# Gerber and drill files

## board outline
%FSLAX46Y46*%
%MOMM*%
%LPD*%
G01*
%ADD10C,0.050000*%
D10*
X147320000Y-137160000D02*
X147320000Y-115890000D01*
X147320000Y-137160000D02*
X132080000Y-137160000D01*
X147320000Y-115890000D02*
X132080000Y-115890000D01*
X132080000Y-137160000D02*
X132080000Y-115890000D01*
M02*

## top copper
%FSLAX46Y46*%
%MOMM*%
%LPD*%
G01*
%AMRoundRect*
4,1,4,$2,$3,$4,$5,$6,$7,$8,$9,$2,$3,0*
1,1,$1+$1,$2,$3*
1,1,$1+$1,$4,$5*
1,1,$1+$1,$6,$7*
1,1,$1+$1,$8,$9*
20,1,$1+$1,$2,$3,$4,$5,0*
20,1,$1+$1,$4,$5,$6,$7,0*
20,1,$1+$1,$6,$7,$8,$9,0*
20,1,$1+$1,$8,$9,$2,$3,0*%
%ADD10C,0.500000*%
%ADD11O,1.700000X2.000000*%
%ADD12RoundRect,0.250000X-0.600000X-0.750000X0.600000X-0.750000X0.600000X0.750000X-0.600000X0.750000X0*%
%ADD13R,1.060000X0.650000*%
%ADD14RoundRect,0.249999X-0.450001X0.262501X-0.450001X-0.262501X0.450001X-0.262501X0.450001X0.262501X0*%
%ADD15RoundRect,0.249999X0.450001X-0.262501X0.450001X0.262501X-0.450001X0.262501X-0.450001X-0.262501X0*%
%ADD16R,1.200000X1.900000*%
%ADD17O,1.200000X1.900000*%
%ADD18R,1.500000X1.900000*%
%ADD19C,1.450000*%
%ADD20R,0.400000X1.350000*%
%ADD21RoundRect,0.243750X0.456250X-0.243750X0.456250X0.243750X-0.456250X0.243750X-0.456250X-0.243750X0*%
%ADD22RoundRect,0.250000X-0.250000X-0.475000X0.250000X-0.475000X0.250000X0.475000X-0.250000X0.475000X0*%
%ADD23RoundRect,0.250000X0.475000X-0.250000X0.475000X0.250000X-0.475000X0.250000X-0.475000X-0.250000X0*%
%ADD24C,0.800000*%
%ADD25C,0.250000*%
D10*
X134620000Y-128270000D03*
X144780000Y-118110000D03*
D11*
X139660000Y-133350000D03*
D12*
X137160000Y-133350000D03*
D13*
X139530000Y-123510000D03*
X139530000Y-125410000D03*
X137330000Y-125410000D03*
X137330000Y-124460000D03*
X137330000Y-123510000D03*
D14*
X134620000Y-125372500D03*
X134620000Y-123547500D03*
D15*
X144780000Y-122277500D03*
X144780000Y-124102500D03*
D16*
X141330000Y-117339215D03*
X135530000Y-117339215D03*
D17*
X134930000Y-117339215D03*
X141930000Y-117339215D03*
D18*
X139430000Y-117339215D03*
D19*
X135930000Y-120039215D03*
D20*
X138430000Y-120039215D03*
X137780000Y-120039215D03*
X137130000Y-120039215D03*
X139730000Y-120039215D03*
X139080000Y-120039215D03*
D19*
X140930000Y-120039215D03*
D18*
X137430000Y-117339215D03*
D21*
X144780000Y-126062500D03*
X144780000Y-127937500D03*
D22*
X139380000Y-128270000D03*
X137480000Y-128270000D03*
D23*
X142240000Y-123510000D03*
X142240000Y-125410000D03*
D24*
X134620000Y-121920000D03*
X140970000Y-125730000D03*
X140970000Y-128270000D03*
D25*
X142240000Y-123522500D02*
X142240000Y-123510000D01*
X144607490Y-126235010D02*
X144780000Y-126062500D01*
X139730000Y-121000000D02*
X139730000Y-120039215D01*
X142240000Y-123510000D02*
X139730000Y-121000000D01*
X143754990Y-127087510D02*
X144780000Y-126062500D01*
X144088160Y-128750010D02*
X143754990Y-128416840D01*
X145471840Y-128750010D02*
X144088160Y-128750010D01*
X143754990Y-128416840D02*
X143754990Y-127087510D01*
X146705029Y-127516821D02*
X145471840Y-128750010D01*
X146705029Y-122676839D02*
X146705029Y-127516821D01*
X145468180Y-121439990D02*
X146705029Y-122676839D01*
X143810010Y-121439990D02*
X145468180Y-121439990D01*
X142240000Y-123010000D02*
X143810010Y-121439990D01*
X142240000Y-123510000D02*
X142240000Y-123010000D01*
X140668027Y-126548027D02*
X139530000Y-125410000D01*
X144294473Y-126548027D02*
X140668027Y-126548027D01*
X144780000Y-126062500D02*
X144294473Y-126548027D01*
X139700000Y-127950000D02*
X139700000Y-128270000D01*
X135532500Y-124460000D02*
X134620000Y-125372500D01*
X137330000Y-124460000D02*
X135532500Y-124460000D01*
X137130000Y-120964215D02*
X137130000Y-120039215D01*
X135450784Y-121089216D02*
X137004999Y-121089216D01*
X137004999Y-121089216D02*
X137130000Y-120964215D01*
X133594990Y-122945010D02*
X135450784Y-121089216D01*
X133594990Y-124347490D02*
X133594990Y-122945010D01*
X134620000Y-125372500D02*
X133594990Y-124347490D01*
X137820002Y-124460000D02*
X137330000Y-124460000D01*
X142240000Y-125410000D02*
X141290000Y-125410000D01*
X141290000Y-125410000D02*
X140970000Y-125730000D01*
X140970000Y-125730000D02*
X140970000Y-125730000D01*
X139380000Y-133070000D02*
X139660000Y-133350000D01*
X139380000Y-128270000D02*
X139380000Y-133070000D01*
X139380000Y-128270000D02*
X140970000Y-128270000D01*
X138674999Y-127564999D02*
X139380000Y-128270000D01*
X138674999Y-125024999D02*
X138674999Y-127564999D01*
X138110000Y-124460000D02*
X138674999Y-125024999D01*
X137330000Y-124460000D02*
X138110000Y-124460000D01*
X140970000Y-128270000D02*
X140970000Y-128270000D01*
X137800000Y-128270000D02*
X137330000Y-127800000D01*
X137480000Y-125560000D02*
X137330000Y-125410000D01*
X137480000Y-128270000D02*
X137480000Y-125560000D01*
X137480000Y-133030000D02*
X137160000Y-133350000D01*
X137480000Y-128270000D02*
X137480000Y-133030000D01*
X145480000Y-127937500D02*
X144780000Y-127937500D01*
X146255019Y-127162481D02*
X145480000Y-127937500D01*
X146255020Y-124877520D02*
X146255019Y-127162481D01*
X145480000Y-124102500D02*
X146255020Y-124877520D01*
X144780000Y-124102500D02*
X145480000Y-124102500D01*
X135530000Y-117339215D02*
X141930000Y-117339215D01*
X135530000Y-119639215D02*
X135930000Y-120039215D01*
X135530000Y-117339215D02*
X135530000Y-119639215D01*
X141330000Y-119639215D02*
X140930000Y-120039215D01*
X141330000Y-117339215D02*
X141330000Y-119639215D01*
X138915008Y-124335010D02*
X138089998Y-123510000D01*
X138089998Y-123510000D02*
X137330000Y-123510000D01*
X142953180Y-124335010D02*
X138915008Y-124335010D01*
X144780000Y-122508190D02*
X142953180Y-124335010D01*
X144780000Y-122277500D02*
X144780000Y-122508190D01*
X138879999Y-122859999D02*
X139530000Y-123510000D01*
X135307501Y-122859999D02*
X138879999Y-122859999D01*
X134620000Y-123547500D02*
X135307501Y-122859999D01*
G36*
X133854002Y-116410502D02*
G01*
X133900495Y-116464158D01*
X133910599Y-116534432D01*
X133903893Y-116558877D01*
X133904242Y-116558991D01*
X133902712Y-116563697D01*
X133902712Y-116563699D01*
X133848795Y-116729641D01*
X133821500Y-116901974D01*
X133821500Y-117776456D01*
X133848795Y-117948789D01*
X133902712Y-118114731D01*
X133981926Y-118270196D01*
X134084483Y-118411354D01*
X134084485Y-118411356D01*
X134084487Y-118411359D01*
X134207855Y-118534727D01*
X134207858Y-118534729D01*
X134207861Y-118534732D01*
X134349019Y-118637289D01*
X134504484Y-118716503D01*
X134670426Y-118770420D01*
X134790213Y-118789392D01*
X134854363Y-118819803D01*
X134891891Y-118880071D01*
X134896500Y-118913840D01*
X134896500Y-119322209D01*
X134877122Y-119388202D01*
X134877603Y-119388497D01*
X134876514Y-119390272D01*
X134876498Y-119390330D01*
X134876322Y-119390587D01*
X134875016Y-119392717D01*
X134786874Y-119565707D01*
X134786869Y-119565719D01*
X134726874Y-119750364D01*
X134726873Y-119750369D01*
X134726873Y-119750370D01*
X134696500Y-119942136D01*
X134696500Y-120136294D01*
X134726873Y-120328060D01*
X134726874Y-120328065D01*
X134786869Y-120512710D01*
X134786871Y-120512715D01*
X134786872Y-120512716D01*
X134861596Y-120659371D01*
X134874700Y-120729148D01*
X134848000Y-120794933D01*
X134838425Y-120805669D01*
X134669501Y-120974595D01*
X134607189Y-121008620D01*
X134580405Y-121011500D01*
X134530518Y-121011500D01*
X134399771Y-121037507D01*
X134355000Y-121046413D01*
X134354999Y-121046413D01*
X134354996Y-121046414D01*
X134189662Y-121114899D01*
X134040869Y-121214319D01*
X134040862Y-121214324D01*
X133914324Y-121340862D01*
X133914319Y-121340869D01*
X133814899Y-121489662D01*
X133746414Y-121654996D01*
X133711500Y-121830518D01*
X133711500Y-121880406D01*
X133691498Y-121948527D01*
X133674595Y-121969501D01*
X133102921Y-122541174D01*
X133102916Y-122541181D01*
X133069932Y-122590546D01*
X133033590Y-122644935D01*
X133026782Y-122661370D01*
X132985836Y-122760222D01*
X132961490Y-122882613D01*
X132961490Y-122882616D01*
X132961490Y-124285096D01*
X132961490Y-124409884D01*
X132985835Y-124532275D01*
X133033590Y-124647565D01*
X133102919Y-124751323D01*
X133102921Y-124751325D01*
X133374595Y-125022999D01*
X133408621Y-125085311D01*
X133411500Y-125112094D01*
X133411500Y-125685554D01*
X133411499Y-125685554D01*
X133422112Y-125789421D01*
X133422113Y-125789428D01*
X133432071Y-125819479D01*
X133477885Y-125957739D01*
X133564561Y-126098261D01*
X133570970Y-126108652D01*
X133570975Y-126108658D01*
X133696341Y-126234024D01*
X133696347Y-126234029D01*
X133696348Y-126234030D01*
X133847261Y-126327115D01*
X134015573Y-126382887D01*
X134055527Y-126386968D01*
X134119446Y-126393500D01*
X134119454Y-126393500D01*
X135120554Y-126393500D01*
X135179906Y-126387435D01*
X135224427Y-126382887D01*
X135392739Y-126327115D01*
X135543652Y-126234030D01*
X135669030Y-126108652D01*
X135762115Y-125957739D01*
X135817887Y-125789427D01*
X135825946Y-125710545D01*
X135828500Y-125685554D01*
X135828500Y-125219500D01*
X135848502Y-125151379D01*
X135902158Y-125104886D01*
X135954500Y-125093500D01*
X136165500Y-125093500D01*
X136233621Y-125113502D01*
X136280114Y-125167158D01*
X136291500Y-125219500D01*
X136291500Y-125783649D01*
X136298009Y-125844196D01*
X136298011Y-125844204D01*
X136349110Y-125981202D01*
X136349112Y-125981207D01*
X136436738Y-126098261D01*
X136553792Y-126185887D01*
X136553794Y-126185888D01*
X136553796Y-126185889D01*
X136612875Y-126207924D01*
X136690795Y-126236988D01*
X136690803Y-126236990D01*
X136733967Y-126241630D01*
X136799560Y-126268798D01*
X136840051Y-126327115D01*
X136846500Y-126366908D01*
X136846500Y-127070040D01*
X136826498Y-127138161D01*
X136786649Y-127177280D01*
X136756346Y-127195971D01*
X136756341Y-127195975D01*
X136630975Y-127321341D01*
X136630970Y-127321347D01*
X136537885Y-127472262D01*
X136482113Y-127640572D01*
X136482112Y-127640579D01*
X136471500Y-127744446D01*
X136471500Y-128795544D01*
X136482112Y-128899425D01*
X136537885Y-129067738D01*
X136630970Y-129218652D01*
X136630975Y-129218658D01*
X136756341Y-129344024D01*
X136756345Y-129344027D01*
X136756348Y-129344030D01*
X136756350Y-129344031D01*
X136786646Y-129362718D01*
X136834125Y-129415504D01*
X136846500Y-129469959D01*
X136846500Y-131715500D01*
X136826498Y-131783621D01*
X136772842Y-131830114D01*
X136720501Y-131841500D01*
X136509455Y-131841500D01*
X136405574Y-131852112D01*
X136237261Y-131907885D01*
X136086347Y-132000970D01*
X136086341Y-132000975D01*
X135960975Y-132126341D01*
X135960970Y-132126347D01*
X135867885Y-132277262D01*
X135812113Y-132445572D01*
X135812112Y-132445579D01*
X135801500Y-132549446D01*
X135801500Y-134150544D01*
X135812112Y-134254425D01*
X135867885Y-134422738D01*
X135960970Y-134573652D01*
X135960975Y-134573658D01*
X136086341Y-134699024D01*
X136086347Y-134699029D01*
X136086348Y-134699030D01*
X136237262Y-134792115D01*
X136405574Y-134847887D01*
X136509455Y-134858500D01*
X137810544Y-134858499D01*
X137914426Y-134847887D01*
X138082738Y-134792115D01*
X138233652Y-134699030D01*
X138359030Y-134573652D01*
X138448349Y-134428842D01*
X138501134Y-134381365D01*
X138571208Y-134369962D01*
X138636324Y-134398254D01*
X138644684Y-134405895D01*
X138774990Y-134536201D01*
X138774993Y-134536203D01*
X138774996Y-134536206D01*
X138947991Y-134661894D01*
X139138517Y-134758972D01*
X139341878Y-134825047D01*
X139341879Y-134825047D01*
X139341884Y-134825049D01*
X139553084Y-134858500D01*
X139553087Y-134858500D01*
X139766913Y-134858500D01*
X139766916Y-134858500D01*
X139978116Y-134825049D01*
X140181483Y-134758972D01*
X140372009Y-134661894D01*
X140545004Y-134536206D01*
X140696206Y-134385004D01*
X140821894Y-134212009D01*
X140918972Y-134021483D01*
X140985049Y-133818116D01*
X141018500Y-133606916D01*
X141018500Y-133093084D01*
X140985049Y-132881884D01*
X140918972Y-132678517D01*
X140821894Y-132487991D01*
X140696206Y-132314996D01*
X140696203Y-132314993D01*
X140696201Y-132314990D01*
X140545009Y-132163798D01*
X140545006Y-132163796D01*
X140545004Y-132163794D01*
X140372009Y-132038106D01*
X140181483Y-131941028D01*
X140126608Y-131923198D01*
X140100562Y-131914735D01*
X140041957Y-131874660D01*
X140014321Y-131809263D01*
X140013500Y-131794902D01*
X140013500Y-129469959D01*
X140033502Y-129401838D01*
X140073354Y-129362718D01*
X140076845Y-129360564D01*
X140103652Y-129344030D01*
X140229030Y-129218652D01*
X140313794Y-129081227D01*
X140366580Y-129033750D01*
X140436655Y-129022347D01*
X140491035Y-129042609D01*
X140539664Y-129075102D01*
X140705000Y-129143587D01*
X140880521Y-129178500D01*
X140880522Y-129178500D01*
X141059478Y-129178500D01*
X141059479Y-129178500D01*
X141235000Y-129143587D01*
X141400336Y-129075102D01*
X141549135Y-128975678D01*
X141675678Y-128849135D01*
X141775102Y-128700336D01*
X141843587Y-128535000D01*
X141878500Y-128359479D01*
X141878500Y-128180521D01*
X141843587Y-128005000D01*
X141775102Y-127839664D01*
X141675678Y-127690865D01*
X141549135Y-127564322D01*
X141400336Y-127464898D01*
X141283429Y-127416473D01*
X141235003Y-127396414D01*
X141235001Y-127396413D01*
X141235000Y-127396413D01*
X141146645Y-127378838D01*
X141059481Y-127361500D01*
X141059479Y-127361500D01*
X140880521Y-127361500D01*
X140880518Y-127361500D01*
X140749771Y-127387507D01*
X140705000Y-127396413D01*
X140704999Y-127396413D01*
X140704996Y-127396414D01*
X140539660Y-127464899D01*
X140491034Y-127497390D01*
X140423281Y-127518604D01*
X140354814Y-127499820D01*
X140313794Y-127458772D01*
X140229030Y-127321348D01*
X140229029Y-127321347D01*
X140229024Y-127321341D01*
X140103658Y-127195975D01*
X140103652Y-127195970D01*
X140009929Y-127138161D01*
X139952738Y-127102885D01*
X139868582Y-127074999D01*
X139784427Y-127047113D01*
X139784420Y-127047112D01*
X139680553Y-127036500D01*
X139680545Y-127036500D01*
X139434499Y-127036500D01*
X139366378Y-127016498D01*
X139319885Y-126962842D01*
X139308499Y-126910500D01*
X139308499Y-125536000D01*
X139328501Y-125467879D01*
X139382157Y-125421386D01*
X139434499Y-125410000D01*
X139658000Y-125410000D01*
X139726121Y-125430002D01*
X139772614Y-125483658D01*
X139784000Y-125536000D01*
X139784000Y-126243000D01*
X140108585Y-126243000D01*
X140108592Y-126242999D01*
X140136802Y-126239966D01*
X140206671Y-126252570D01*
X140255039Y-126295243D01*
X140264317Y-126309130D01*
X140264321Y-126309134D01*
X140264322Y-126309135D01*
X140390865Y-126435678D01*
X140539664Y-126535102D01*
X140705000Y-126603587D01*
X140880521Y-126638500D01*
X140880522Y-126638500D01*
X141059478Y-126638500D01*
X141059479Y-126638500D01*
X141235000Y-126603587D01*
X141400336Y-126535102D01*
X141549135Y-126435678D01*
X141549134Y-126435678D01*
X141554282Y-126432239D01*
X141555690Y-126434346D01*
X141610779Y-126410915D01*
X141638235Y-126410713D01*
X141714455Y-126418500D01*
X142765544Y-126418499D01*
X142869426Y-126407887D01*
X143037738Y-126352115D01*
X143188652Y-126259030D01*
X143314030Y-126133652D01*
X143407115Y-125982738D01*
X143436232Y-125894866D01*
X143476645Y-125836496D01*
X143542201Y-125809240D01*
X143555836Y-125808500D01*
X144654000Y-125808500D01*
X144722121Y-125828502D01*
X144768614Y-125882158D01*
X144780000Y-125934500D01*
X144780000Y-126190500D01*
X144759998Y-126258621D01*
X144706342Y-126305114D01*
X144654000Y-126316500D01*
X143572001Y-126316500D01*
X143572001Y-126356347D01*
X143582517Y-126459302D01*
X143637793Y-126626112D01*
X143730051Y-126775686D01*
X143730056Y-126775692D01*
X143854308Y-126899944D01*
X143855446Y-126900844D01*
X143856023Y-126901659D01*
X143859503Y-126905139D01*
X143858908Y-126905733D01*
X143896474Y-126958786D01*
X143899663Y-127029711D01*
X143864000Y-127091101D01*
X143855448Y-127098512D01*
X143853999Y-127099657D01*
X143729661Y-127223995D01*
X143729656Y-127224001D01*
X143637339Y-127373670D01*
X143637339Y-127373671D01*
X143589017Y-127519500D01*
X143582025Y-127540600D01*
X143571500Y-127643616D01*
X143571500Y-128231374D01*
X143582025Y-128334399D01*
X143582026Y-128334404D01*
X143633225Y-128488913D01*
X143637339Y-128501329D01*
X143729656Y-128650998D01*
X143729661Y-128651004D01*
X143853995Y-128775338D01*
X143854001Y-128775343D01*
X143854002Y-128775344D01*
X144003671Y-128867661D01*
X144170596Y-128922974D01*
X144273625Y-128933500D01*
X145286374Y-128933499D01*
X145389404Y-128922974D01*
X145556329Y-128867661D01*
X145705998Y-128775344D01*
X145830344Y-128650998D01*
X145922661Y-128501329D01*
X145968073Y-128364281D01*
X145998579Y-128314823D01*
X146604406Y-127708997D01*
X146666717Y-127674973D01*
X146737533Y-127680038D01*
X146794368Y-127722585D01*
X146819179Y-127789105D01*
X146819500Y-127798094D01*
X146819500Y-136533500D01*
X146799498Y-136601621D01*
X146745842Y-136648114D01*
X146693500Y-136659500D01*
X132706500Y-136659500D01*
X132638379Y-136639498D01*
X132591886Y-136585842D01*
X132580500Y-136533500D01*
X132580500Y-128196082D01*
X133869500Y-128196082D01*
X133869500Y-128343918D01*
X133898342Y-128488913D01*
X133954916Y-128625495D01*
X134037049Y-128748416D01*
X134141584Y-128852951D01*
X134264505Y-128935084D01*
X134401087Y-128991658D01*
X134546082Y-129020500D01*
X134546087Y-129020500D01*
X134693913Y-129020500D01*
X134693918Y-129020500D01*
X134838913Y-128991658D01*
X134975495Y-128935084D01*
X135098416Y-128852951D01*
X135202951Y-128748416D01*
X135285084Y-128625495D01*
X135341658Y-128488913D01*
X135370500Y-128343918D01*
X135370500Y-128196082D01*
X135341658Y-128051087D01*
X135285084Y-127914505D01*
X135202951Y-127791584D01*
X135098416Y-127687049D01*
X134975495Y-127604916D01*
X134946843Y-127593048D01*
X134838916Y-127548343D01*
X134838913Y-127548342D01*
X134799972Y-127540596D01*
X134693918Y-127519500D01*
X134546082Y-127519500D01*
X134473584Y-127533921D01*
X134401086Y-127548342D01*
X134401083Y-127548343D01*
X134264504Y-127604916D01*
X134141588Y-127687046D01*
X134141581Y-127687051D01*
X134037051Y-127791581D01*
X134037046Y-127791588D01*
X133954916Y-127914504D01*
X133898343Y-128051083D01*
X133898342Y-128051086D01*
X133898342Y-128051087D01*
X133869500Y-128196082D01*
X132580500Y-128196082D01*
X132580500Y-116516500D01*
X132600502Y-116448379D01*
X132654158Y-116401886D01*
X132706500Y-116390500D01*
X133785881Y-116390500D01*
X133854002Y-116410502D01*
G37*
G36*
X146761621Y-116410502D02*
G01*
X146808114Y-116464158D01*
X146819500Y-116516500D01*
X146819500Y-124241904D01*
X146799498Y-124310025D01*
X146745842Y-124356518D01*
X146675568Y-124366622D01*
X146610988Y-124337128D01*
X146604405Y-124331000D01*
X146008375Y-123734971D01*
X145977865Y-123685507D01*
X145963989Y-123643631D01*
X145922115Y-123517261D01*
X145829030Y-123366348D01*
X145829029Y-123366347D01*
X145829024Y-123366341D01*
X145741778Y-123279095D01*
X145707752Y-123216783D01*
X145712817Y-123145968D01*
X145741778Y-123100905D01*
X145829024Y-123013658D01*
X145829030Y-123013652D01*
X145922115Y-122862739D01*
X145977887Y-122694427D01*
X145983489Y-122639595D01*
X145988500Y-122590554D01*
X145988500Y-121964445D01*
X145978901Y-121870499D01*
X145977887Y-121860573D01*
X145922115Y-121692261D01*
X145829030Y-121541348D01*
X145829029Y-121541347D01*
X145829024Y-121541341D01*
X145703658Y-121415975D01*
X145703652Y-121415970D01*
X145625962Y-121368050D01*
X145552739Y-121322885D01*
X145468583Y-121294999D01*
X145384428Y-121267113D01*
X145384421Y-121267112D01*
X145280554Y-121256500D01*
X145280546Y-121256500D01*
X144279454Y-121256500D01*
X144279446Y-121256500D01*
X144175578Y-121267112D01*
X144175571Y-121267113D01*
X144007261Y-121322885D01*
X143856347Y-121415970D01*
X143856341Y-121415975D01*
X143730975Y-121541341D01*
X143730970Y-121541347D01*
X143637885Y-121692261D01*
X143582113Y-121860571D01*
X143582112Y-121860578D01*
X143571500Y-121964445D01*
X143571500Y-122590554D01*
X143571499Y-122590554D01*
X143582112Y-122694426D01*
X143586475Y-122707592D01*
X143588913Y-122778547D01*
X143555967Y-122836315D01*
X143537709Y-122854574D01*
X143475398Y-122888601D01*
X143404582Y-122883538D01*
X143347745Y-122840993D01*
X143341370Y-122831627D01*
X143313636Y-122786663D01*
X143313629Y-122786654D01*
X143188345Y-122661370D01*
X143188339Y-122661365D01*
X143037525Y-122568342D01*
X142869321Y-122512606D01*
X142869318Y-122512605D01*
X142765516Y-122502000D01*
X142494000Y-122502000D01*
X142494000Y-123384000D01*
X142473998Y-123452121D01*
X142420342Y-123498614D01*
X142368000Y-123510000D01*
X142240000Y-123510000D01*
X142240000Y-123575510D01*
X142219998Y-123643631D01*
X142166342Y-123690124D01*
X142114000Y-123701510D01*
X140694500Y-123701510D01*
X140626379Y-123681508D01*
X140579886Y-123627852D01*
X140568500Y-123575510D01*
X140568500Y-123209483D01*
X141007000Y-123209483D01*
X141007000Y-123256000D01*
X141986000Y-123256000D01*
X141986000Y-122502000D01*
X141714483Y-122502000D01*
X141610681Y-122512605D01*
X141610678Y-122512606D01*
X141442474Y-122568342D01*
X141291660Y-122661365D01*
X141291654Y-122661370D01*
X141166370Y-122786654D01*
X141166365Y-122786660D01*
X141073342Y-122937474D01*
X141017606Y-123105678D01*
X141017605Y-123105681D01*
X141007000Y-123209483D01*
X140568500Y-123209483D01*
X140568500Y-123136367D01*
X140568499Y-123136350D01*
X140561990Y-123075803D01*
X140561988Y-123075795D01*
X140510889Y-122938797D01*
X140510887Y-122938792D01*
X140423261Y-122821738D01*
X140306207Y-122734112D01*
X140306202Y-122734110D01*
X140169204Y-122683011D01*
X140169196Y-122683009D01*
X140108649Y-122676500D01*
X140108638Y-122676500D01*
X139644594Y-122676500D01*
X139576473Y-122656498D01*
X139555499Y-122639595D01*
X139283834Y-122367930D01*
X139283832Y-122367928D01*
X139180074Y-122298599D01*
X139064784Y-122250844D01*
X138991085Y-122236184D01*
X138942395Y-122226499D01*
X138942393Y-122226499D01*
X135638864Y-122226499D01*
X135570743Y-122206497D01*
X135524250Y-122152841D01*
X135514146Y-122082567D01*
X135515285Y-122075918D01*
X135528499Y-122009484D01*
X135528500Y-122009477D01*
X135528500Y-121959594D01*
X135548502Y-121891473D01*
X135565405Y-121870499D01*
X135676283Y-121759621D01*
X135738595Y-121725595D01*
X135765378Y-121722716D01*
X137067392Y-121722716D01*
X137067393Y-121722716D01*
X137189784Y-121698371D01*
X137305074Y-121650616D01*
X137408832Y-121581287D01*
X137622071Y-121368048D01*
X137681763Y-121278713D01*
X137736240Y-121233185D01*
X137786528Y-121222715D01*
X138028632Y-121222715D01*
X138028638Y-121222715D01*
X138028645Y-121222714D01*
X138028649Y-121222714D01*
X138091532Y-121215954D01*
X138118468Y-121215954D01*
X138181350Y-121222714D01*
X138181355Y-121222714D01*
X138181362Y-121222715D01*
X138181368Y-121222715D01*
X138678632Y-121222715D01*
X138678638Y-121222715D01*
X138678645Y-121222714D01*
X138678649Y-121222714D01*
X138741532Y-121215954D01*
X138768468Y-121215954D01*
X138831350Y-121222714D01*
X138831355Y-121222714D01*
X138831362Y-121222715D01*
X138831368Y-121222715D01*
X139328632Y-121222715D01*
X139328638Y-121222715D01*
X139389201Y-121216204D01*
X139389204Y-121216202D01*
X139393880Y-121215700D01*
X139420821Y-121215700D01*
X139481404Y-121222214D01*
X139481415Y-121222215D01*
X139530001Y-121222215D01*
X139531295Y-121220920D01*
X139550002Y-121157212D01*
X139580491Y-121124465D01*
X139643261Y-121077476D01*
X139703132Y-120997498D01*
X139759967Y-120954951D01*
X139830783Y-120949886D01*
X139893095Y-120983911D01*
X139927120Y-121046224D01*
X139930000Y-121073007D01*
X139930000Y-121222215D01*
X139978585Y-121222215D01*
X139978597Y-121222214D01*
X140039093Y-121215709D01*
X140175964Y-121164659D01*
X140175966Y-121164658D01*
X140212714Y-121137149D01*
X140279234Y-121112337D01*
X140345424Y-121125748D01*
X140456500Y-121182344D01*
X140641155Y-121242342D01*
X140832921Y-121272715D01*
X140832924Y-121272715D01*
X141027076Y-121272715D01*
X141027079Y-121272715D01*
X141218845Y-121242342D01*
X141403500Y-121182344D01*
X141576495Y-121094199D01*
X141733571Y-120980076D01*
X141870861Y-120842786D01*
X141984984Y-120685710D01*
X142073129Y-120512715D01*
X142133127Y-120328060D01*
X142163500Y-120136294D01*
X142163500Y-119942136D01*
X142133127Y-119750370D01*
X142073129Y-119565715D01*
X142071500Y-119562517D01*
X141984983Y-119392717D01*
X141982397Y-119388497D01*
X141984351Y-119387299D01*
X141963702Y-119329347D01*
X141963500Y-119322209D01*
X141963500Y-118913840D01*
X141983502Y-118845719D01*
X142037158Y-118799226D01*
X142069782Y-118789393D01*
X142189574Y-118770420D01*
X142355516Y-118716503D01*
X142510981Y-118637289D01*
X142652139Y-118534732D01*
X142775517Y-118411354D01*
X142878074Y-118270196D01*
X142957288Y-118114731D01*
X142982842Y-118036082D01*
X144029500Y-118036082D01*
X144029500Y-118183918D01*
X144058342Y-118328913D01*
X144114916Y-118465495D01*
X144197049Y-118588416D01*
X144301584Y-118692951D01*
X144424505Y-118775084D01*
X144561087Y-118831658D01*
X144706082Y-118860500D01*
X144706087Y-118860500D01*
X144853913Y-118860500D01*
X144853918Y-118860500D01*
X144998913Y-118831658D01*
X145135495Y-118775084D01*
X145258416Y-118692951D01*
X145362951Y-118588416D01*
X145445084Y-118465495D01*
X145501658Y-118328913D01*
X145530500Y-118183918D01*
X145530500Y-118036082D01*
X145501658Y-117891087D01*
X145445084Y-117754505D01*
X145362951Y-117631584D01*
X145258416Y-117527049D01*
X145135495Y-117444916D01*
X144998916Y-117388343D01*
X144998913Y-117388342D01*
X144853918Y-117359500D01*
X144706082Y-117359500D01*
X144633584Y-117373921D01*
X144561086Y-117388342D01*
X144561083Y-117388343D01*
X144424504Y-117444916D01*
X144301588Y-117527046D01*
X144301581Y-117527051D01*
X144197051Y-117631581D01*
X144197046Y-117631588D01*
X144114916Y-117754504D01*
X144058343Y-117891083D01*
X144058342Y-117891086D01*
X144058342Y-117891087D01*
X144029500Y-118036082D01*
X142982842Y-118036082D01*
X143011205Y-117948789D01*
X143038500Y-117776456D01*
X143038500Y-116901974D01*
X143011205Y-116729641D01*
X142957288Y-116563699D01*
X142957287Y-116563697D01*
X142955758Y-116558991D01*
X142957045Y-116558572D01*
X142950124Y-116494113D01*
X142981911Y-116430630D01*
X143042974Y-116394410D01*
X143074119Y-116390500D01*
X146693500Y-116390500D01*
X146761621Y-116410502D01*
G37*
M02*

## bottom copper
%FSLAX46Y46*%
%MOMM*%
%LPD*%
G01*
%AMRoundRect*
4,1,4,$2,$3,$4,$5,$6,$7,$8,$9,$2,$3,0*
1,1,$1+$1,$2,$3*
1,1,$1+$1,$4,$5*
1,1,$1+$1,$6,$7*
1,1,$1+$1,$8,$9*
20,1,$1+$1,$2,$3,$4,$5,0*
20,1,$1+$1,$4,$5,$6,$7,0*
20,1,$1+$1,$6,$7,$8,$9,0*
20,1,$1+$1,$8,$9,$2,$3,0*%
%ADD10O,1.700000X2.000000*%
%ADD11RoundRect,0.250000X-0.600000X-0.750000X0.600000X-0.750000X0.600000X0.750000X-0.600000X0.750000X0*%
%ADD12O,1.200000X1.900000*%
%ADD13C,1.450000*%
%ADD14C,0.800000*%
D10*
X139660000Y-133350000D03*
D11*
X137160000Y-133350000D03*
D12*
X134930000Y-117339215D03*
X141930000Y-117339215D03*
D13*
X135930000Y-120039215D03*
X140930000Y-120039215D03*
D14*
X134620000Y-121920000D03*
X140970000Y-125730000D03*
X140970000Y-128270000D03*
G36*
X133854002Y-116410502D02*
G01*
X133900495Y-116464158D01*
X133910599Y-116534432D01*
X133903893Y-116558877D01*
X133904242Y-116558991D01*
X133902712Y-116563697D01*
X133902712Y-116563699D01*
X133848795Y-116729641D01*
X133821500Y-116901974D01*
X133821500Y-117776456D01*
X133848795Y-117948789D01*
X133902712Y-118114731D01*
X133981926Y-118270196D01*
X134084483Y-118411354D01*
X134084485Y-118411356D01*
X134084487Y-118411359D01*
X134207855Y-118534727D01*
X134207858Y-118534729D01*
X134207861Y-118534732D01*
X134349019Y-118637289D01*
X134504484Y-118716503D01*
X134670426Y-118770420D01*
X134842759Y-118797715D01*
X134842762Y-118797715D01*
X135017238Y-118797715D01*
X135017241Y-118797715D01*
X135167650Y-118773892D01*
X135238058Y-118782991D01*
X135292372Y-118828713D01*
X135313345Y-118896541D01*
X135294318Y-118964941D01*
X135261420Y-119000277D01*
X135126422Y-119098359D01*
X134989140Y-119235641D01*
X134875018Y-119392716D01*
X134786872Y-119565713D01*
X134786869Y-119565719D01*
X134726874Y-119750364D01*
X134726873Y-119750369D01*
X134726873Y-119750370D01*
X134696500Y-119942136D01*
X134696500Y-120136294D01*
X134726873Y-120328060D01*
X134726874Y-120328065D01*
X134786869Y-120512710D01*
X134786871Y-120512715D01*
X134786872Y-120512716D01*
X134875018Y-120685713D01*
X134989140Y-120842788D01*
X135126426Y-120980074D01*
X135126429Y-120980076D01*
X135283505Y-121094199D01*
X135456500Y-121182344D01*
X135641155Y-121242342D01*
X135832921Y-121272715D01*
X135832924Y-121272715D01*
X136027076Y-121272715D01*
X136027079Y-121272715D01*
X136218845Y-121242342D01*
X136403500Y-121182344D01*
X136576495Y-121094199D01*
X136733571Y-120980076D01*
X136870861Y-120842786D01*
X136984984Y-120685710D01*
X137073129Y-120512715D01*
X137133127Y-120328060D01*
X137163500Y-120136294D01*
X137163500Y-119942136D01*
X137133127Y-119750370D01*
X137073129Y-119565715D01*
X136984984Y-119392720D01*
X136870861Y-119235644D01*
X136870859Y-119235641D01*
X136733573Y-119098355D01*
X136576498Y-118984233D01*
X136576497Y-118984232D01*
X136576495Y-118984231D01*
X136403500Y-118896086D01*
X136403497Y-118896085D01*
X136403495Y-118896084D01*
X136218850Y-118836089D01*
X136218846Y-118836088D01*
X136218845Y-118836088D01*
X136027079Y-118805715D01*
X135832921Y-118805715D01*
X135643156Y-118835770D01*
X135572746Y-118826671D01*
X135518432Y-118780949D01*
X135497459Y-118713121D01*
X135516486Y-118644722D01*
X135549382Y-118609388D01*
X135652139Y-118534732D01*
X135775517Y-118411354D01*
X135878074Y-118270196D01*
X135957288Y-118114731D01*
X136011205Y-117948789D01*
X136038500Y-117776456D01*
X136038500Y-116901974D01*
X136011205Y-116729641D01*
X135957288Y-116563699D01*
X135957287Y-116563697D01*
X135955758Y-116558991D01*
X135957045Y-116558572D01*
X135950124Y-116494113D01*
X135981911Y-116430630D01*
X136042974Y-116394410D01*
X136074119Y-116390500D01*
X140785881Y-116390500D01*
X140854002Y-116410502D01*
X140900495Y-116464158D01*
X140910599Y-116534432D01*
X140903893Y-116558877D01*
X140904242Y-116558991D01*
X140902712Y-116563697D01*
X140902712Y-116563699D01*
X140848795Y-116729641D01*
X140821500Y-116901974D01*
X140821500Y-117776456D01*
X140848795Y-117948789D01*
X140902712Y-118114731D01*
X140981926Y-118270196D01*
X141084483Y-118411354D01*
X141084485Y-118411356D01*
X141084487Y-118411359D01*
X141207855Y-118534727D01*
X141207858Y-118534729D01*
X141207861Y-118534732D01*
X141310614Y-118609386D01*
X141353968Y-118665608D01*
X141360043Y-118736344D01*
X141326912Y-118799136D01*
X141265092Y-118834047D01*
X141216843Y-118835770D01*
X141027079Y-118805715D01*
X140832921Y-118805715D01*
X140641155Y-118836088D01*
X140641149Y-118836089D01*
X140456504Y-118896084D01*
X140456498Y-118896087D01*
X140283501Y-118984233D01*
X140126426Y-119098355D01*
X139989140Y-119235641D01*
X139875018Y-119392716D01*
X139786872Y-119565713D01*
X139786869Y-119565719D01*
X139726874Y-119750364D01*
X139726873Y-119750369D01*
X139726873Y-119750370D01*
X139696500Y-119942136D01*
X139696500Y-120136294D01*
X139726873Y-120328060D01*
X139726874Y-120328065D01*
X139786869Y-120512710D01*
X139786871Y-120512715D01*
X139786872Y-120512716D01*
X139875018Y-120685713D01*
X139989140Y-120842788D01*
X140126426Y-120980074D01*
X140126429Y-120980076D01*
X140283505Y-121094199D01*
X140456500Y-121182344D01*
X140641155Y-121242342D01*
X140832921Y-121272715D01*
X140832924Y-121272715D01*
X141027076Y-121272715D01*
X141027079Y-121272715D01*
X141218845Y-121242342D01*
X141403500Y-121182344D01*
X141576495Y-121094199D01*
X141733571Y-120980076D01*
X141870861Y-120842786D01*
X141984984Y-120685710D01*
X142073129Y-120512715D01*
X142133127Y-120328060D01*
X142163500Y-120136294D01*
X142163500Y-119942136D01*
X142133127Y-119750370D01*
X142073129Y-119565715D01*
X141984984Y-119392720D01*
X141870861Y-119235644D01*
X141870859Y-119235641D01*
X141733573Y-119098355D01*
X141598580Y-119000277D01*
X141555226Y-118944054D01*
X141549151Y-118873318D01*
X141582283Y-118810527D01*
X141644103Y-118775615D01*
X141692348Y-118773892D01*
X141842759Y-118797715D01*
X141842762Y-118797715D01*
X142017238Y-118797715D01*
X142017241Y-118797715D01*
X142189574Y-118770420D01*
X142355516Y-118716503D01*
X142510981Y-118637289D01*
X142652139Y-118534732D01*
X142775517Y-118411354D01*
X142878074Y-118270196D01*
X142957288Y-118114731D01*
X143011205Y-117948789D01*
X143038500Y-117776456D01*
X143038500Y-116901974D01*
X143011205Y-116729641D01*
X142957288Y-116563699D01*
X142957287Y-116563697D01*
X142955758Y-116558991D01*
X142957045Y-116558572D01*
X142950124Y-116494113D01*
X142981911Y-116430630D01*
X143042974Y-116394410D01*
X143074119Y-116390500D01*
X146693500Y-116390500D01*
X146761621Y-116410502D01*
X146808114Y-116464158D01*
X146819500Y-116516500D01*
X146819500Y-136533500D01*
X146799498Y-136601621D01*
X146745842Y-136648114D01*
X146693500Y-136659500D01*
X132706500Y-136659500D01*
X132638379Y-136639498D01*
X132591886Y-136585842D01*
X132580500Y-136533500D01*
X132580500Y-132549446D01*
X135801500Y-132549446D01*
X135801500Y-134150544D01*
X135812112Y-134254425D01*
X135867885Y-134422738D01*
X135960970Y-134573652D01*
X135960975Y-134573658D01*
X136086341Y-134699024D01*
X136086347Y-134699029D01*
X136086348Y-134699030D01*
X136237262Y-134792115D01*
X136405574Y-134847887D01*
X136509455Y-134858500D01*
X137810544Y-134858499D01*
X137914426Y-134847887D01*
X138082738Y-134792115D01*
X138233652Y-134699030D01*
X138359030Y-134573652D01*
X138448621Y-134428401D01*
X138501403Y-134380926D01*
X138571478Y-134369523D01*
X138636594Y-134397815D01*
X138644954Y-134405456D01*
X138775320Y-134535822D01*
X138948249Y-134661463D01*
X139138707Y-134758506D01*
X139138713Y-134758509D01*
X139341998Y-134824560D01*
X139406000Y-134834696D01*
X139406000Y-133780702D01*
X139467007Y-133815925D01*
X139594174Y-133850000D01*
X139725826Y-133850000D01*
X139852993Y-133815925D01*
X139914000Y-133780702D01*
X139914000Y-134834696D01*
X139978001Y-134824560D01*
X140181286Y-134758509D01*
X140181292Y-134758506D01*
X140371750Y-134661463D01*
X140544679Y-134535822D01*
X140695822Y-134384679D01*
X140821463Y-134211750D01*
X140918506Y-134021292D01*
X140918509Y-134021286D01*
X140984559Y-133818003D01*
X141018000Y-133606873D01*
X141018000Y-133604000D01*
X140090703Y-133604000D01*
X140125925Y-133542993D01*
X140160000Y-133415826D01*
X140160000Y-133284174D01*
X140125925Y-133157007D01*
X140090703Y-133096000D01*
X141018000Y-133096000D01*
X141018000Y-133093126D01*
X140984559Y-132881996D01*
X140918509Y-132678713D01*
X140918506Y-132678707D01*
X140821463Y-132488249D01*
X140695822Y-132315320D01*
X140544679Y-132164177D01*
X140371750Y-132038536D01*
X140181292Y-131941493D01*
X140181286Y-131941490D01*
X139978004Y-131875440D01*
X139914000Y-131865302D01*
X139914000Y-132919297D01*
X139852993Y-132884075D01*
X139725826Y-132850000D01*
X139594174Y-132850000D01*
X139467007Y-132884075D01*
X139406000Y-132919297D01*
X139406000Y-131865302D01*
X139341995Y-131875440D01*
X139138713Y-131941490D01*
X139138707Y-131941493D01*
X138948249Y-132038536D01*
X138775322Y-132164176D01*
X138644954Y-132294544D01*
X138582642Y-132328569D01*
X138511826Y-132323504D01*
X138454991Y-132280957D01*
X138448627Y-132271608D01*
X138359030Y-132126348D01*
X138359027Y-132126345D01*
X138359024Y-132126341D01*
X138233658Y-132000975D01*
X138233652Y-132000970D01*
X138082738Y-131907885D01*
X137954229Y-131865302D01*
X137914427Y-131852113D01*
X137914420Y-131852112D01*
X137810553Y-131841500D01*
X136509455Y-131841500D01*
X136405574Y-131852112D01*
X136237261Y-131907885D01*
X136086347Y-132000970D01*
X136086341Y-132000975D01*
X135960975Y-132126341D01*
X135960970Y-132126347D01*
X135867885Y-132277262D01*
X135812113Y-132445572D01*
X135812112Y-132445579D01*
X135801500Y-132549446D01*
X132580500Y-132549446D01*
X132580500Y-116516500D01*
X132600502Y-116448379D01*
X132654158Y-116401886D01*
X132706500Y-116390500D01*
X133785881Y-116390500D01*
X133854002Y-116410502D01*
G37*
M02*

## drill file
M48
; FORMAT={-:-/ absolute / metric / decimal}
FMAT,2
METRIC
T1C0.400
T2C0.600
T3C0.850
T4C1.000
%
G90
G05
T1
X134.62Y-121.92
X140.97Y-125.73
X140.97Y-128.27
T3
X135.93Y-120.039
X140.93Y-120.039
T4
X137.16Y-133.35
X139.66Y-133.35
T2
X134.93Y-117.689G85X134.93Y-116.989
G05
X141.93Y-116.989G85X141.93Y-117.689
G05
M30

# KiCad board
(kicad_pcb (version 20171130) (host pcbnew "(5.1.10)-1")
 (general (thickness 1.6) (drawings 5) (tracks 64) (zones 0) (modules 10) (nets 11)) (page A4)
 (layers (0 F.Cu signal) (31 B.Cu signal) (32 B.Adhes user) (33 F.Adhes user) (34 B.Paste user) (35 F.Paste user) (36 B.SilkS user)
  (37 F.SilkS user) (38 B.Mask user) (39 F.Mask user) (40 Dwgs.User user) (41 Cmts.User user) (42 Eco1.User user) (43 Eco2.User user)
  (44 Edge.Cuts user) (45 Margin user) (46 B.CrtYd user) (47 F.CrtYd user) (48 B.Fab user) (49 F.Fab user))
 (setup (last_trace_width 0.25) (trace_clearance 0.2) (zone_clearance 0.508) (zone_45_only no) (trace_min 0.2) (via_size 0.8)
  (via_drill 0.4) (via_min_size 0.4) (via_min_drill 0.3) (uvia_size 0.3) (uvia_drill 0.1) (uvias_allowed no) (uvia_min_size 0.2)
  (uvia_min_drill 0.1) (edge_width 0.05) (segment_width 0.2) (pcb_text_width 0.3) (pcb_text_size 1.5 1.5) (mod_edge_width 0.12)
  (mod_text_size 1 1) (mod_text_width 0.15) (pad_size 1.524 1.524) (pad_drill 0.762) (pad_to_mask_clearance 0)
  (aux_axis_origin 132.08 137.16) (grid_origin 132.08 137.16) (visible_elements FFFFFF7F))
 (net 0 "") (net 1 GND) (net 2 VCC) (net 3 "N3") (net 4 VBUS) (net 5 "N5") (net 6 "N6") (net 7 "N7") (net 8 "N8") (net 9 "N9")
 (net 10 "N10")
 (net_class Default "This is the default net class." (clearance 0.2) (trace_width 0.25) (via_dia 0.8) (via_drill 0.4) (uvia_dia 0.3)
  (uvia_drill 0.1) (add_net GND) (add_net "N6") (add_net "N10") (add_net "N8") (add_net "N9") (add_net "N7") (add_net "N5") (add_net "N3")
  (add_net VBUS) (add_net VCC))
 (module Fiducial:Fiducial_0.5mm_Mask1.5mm (layer F.Cu) (at 134.62 128.27)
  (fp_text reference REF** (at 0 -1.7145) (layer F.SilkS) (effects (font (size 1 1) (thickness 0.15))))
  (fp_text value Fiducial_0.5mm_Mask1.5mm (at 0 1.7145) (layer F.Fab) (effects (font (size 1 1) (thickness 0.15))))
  (pad "" smd circle (at 0 0) (size 0.5 0.5) (layers F.Cu F.Mask) (solder_mask_margin 0.5) (clearance 0.5)))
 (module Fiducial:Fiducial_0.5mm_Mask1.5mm (layer F.Cu) (at 144.78 118.11)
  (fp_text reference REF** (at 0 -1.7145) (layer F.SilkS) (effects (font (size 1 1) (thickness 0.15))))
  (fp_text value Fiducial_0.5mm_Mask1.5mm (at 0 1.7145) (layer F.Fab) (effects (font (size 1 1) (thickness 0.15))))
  (pad "" smd circle (at 0 0) (size 0.5 0.5) (layers F.Cu F.Mask) (solder_mask_margin 0.5) (clearance 0.5)))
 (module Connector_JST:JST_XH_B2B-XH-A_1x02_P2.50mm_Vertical (layer F.Cu) (at 137.16 133.35)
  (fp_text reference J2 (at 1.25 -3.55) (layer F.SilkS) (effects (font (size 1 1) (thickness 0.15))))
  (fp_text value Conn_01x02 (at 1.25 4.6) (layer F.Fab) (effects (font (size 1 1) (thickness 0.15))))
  (pad 2 thru_hole oval (at 2.5 0) (size 1.7 2) (drill 1) (layers *.Cu *.Mask) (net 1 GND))
  (pad 1 thru_hole roundrect (at 0 0) (size 1.7 2) (drill 1) (layers *.Cu *.Mask) (roundrect_rratio 0.1470588235294118) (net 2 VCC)))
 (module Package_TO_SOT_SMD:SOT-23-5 (layer F.Cu) (at 138.43 124.46)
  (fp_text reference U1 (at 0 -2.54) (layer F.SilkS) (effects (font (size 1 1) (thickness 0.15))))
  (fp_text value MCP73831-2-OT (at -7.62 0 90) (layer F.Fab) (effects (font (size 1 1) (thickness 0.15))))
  (pad 5 smd rect (at 1.1 -0.95) (size 1.06 0.65) (layers F.Cu F.Paste F.Mask) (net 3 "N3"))
  (pad 4 smd rect (at 1.1 0.95) (size 1.06 0.65) (layers F.Cu F.Paste F.Mask) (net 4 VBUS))
  (pad 3 smd rect (at -1.1 0.95) (size 1.06 0.65) (layers F.Cu F.Paste F.Mask) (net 2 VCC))
  (pad 2 smd rect (at -1.1 0) (size 1.06 0.65) (layers F.Cu F.Paste F.Mask) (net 1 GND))
  (pad 1 smd rect (at -1.1 -0.95) (size 1.06 0.65) (layers F.Cu F.Paste F.Mask) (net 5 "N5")))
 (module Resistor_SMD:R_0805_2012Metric (layer F.Cu) (at 134.62 124.46 270)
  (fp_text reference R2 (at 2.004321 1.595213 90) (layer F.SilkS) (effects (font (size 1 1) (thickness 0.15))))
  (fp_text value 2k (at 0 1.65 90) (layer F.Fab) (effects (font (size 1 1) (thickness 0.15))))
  (pad 2 smd roundrect (at 0.9125 0 270) (size 1.025 1.4) (layers F.Cu F.Paste F.Mask) (roundrect_rratio 0.2439014634146341) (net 1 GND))
  (pad 1 smd roundrect (at -0.9125 0 270) (size 1.025 1.4) (layers F.Cu F.Paste F.Mask) (roundrect_rratio 0.2439014634146341) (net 3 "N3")))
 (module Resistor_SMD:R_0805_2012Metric (layer F.Cu) (at 144.78 123.19 90)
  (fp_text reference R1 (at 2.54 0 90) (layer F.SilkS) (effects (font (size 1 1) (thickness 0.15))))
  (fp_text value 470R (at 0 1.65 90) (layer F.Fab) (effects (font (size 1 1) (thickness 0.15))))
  (pad 2 smd roundrect (at 0.9125 0 90) (size 1.025 1.4) (layers F.Cu F.Paste F.Mask) (roundrect_rratio 0.2439014634146341) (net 5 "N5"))
  (pad 1 smd roundrect (at -0.9125 0 90) (size 1.025 1.4) (layers F.Cu F.Paste F.Mask) (roundrect_rratio 0.2439014634146341) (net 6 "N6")))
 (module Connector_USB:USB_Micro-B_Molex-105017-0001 (layer F.Cu) (at 138.43 118.576715 180)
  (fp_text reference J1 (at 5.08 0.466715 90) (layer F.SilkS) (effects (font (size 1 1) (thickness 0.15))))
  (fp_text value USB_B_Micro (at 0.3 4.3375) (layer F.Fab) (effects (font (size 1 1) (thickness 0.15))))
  (pad 6 smd rect (at -2.9 1.2375 180) (size 1.2 1.9) (layers F.Cu F.Mask) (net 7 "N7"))
  (pad 6 smd rect (at 2.9 1.2375 180) (size 1.2 1.9) (layers F.Cu F.Mask) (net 7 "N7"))
  (pad 6 thru_hole oval (at 3.5 1.2375 180) (size 1.2 1.9) (drill oval 0.6 1.3) (layers *.Cu *.Mask) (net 7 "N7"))
  (pad 6 thru_hole oval (at -3.5 1.2375) (size 1.2 1.9) (drill oval 0.6 1.3) (layers *.Cu *.Mask) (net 7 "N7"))
  (pad 6 smd rect (at -1 1.2375 180) (size 1.5 1.9) (layers F.Cu F.Paste F.Mask) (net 7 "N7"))
  (pad 6 thru_hole circle (at 2.5 -1.4625 180) (size 1.45 1.45) (drill 0.85) (layers *.Cu *.Mask) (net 7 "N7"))
  (pad 3 smd rect (at 0 -1.4625 180) (size 0.4 1.35) (layers F.Cu F.Paste F.Mask) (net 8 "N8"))
  (pad 4 smd rect (at 0.65 -1.4625 180) (size 0.4 1.35) (layers F.Cu F.Paste F.Mask) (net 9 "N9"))
  (pad 5 smd rect (at 1.3 -1.4625 180) (size 0.4 1.35) (layers F.Cu F.Paste F.Mask) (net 1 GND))
  (pad 1 smd rect (at -1.3 -1.4625 180) (size 0.4 1.35) (layers F.Cu F.Paste F.Mask) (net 4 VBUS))
  (pad 2 smd rect (at -0.65 -1.4625 180) (size 0.4 1.35) (layers F.Cu F.Paste F.Mask) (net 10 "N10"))
  (pad 6 thru_hole circle (at -2.5 -1.4625 180) (size 1.45 1.45) (drill 0.85) (layers *.Cu *.Mask) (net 7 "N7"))
  (pad 6 smd rect (at 1 1.2375 180) (size 1.5 1.9) (layers F.Cu F.Paste F.Mask) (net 7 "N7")))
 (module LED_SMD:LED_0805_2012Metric (layer F.Cu) (at 144.78 127 90)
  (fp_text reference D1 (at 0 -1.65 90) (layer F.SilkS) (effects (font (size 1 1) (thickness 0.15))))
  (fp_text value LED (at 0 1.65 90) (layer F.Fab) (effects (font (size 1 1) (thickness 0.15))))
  (pad 2 smd roundrect (at 0.9375 0 90) (size 0.975 1.4) (layers F.Cu F.Paste F.Mask) (roundrect_rratio 0.25) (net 4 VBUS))
  (pad 1 smd roundrect (at -0.9375 0 90) (size 0.975 1.4) (layers F.Cu F.Paste F.Mask) (roundrect_rratio 0.25) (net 6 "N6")))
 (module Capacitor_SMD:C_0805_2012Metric (layer F.Cu) (at 138.43 128.27)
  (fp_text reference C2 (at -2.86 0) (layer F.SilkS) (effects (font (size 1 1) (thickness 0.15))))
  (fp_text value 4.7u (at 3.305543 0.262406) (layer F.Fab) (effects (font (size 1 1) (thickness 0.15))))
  (pad 2 smd roundrect (at 0.95 0) (size 1 1.45) (layers F.Cu F.Paste F.Mask) (roundrect_rratio 0.25) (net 1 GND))
  (pad 1 smd roundrect (at -0.95 0) (size 1 1.45) (layers F.Cu F.Paste F.Mask) (roundrect_rratio 0.25) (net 2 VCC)))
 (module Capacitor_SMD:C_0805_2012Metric (layer F.Cu) (at 142.24 124.46 90)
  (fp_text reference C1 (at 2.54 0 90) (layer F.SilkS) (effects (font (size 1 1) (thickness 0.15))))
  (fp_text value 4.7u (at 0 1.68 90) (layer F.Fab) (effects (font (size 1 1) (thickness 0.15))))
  (pad 2 smd roundrect (at 0.95 0 90) (size 1 1.45) (layers F.Cu F.Paste F.Mask) (roundrect_rratio 0.25) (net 4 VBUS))
  (pad 1 smd roundrect (at -0.95 0 90) (size 1 1.45) (layers F.Cu F.Paste F.Mask) (roundrect_rratio 0.25) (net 1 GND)))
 (gr_line (start 147.32 137.16) (end 147.32 115.89) (layer Edge.Cuts) (width 0.05))
 (gr_line (start 147.32 137.16) (end 132.08 137.16) (layer Edge.Cuts) (width 0.05))
 (gr_line (start 147.32 115.89) (end 132.08 115.89) (layer Edge.Cuts) (width 0.05))
 (gr_line (start 132.08 137.16) (end 132.08 115.89) (layer Edge.Cuts) (width 0.05))
 (via (at 134.62 121.92) (size 0.8) (drill 0.4) (layers F.Cu B.Cu) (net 1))
 (segment (start 142.24 123.5225) (end 142.24 123.51) (width 0.25) (layer F.Cu) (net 4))
 (segment (start 144.60749 126.23501) (end 144.78 126.0625) (width 0.25) (layer F.Cu) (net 4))
 (segment (start 139.73 121) (end 139.73 120.039215) (width 0.25) (layer F.Cu) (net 4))
 (segment (start 142.24 123.51) (end 139.73 121) (width 0.25) (layer F.Cu) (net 4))
 (segment (start 143.75499 127.08751) (end 144.78 126.0625) (width 0.25) (layer F.Cu) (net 4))
 (segment (start 144.08816 128.75001) (end 143.75499 128.41684) (width 0.25) (layer F.Cu) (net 4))
 (segment (start 145.47184 128.75001) (end 144.08816 128.75001) (width 0.25) (layer F.Cu) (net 4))
 (segment (start 143.75499 128.41684) (end 143.75499 127.08751) (width 0.25) (layer F.Cu) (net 4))
 (segment (start 146.705029 127.516821) (end 145.47184 128.75001) (width 0.25) (layer F.Cu) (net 4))
 (segment (start 146.705029 122.676839) (end 146.705029 127.516821) (width 0.25) (layer F.Cu) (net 4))
 (segment (start 145.46818 121.43999) (end 146.705029 122.676839) (width 0.25) (layer F.Cu) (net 4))
 (segment (start 143.81001 121.43999) (end 145.46818 121.43999) (width 0.25) (layer F.Cu) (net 4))
 (segment (start 142.24 123.01) (end 143.81001 121.43999) (width 0.25) (layer F.Cu) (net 4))
 (segment (start 142.24 123.51) (end 142.24 123.01) (width 0.25) (layer F.Cu) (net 4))
 (segment (start 140.668027 126.548027) (end 139.53 125.41) (width 0.25) (layer F.Cu) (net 4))
 (segment (start 144.294473 126.548027) (end 140.668027 126.548027) (width 0.25) (layer F.Cu) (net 4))
 (segment (start 144.78 126.0625) (end 144.294473 126.548027) (width 0.25) (layer F.Cu) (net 4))
 (segment (start 139.7 127.95) (end 139.7 128.27) (width 0.25) (layer F.Cu) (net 1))
 (segment (start 135.5325 124.46) (end 134.62 125.3725) (width 0.25) (layer F.Cu) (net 1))
 (segment (start 137.33 124.46) (end 135.5325 124.46) (width 0.25) (layer F.Cu) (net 1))
 (segment (start 137.13 120.964215) (end 137.13 120.039215) (width 0.25) (layer F.Cu) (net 1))
 (segment (start 135.450784 121.089216) (end 137.004999 121.089216) (width 0.25) (layer F.Cu) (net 1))
 (segment (start 137.004999 121.089216) (end 137.13 120.964215) (width 0.25) (layer F.Cu) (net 1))
 (segment (start 133.59499 122.94501) (end 135.450784 121.089216) (width 0.25) (layer F.Cu) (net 1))
 (segment (start 133.59499 124.34749) (end 133.59499 122.94501) (width 0.25) (layer F.Cu) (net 1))
 (segment (start 134.62 125.3725) (end 133.59499 124.34749) (width 0.25) (layer F.Cu) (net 1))
 (segment (start 137.820002 124.46) (end 137.33 124.46) (width 0.25) (layer F.Cu) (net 1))
 (segment (start 142.24 125.41) (end 141.29 125.41) (width 0.25) (layer F.Cu) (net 1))
 (segment (start 141.29 125.41) (end 140.97 125.73) (width 0.25) (layer F.Cu) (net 1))
 (segment (start 140.97 125.73) (end 140.97 125.73) (width 0.25) (layer F.Cu) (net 1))
 (via (at 140.97 125.73) (size 0.8) (drill 0.4) (layers F.Cu B.Cu) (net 1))
 (segment (start 139.38 133.07) (end 139.66 133.35) (width 0.25) (layer F.Cu) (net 1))
 (segment (start 139.38 128.27) (end 139.38 133.07) (width 0.25) (layer F.Cu) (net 1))
 (segment (start 139.38 128.27) (end 140.97 128.27) (width 0.25) (layer F.Cu) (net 1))
 (segment (start 138.674999 127.564999) (end 139.38 128.27) (width 0.25) (layer F.Cu) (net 1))
 (segment (start 138.674999 125.024999) (end 138.674999 127.564999) (width 0.25) (layer F.Cu) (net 1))
 (segment (start 138.11 124.46) (end 138.674999 125.024999) (width 0.25) (layer F.Cu) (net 1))
 (segment (start 137.33 124.46) (end 138.11 124.46) (width 0.25) (layer F.Cu) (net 1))
 (segment (start 140.97 128.27) (end 140.97 128.27) (width 0.25) (layer F.Cu) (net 1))
 (via (at 140.97 128.27) (size 0.8) (drill 0.4) (layers F.Cu B.Cu) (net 1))
 (segment (start 137.8 128.27) (end 137.33 127.8) (width 0.25) (layer F.Cu) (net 2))
 (segment (start 137.48 125.56) (end 137.33 125.41) (width 0.25) (layer F.Cu) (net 2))
 (segment (start 137.48 128.27) (end 137.48 125.56) (width 0.25) (layer F.Cu) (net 2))
 (segment (start 137.48 133.03) (end 137.16 133.35) (width 0.25) (layer F.Cu) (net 2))
 (segment (start 137.48 128.27) (end 137.48 133.03) (width 0.25) (layer F.Cu) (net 2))
 (segment (start 145.48 127.9375) (end 144.78 127.9375) (width 0.25) (layer F.Cu) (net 6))
 (segment (start 146.255019 127.162481) (end 145.48 127.9375) (width 0.25) (layer F.Cu) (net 6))
 (segment (start 146.25502 124.87752) (end 146.255019 127.162481) (width 0.25) (layer F.Cu) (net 6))
 (segment (start 145.48 124.1025) (end 146.25502 124.87752) (width 0.25) (layer F.Cu) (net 6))
 (segment (start 144.78 124.1025) (end 145.48 124.1025) (width 0.25) (layer F.Cu) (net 6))
 (segment (start 135.53 117.339215) (end 141.93 117.339215) (width 0.25) (layer F.Cu) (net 7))
 (segment (start 135.53 119.639215) (end 135.93 120.039215) (width 0.25) (layer F.Cu) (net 7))
 (segment (start 135.53 117.339215) (end 135.53 119.639215) (width 0.25) (layer F.Cu) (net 7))
 (segment (start 141.33 119.639215) (end 140.93 120.039215) (width 0.25) (layer F.Cu) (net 7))
 (segment (start 141.33 117.339215) (end 141.33 119.639215) (width 0.25) (layer F.Cu) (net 7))
 (segment (start 138.915008 124.33501) (end 138.089998 123.51) (width 0.25) (layer F.Cu) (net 5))
 (segment (start 138.089998 123.51) (end 137.33 123.51) (width 0.25) (layer F.Cu) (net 5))
 (segment (start 142.95318 124.33501) (end 138.915008 124.33501) (width 0.25) (layer F.Cu) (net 5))
 (segment (start 144.78 122.50819) (end 142.95318 124.33501) (width 0.25) (layer F.Cu) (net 5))
 (segment (start 144.78 122.2775) (end 144.78 122.50819) (width 0.25) (layer F.Cu) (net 5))
 (segment (start 138.879999 122.859999) (end 139.53 123.51) (width 0.25) (layer F.Cu) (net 3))
 (segment (start 135.307501 122.859999) (end 138.879999 122.859999) (width 0.25) (layer F.Cu) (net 3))
 (segment (start 134.62 123.5475) (end 135.307501 122.859999) (width 0.25) (layer F.Cu) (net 3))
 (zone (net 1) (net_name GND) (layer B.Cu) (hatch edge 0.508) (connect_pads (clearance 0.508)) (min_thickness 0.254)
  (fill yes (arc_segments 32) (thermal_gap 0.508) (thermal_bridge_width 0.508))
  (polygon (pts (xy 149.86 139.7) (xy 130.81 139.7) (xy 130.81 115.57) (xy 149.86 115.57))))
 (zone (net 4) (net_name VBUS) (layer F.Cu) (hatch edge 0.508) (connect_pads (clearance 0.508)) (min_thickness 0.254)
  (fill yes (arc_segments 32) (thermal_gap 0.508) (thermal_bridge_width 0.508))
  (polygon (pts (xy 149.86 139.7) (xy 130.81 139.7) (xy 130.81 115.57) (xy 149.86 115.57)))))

